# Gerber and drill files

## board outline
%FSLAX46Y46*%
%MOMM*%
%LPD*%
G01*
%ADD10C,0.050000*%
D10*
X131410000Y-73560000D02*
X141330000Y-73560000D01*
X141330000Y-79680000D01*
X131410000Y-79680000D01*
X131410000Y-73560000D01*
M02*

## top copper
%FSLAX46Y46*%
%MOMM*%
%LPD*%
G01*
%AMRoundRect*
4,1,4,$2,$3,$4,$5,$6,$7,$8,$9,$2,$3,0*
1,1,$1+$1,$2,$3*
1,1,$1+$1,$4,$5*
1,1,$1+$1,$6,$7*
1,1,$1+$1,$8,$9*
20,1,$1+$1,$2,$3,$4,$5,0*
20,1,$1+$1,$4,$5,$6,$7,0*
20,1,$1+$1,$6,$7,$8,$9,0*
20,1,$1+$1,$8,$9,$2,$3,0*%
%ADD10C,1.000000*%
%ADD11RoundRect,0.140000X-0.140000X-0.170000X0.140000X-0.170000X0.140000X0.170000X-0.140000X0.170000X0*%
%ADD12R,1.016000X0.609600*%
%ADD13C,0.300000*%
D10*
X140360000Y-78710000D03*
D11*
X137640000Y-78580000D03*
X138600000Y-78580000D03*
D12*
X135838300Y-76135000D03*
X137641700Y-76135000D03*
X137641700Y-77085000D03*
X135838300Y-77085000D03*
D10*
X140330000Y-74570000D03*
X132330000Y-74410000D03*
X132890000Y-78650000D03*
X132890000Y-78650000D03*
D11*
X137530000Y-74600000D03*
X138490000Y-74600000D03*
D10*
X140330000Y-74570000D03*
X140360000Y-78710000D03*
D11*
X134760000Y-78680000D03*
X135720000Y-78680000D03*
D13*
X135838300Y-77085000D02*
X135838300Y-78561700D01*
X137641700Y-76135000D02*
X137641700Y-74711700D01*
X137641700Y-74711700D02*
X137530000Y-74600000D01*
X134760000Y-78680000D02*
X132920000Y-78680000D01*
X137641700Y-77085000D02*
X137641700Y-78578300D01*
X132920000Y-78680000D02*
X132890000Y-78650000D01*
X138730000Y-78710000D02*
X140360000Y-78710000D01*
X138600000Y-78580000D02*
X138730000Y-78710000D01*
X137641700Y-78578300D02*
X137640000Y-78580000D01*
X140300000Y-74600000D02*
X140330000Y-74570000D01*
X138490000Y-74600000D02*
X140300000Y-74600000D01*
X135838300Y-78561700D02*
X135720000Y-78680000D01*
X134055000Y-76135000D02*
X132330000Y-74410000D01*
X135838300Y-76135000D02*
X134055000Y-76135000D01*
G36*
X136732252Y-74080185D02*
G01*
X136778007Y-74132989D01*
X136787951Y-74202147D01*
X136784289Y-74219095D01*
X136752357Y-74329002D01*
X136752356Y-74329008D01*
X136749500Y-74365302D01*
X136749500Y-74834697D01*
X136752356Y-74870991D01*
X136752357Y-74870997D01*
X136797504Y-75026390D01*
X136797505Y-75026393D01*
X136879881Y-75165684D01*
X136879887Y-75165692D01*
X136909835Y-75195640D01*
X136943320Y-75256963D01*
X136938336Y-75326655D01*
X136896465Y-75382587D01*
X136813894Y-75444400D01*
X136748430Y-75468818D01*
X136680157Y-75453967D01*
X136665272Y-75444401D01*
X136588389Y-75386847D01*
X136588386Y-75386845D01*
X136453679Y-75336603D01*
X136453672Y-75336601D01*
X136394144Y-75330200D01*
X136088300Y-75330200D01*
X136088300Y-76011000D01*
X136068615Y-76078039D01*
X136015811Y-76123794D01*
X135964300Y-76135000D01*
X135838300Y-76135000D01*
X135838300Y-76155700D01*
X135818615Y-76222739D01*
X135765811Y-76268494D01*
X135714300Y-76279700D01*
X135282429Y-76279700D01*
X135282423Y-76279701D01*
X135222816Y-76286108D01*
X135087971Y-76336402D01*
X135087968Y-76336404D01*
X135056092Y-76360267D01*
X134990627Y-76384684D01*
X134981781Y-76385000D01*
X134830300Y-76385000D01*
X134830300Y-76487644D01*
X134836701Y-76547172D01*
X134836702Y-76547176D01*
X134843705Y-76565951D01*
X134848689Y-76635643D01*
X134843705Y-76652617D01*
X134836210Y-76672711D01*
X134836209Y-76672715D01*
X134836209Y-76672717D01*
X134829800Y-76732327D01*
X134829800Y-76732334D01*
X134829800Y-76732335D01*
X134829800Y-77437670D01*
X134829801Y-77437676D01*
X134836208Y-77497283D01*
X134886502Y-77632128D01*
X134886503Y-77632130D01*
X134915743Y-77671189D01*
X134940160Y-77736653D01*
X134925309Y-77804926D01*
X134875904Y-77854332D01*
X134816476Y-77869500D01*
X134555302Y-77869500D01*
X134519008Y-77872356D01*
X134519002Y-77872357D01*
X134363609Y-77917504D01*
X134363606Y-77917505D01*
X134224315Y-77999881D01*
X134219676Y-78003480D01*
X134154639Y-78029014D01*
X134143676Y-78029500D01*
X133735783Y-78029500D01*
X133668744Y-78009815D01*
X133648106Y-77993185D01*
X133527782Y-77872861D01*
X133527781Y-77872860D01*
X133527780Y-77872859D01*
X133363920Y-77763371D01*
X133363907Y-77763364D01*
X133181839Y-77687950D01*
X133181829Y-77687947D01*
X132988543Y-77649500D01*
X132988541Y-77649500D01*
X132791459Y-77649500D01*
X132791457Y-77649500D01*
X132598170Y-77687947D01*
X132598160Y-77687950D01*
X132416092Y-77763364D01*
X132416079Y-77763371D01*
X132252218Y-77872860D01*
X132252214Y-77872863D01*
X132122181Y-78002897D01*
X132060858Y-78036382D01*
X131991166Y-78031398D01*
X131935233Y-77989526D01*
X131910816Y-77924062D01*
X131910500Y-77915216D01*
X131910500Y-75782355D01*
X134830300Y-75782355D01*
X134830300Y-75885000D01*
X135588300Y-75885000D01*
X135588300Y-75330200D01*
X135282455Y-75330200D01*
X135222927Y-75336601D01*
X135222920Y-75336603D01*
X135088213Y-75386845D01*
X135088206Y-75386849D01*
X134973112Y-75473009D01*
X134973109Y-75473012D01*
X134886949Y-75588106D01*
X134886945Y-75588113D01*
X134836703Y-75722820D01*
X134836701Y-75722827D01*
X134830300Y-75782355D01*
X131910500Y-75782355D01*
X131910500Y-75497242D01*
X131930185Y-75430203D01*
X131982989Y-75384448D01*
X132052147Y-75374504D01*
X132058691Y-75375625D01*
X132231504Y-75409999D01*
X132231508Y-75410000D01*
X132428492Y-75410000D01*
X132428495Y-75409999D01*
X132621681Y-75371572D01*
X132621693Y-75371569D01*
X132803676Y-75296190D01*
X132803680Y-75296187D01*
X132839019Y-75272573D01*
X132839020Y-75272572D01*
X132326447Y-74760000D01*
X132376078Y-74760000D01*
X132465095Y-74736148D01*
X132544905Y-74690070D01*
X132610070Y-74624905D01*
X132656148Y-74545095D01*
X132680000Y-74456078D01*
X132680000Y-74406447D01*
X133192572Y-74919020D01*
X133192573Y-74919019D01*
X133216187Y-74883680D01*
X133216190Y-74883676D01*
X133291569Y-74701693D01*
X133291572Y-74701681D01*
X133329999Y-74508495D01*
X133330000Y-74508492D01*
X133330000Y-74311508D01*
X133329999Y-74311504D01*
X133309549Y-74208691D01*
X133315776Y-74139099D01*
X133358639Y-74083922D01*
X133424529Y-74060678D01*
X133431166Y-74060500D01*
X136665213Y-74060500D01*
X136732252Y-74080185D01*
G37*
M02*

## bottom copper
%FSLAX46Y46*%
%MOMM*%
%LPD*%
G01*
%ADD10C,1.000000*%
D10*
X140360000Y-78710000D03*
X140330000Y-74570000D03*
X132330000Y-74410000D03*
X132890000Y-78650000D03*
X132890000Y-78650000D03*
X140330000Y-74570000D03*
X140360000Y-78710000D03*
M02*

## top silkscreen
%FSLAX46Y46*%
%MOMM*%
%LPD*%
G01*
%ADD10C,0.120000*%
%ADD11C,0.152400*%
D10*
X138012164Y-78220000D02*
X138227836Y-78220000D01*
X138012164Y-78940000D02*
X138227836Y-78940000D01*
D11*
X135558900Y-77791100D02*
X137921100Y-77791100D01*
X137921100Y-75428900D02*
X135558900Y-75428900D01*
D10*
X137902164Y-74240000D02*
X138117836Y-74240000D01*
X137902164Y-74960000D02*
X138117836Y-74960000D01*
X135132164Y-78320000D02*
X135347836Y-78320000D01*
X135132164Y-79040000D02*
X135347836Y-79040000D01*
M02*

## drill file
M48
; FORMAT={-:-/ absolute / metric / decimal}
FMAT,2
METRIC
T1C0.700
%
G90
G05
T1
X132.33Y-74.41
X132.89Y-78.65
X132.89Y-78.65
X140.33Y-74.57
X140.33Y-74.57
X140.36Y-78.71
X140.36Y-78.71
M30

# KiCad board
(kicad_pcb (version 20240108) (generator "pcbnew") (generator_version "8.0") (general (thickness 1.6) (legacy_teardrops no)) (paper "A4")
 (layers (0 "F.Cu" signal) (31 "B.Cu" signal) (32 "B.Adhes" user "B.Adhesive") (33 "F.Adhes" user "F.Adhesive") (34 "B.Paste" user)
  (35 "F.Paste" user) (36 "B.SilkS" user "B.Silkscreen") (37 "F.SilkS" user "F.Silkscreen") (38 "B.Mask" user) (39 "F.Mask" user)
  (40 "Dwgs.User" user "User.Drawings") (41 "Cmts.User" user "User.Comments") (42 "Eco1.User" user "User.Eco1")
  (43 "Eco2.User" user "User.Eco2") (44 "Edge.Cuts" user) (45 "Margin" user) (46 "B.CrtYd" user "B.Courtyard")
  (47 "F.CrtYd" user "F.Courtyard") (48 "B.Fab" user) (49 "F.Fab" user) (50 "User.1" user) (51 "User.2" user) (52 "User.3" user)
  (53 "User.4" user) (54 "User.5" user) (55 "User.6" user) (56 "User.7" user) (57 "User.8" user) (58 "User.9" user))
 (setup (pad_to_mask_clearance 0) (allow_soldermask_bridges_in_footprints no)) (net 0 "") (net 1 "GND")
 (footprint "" (layer "F.Cu") (at 140.36 78.71)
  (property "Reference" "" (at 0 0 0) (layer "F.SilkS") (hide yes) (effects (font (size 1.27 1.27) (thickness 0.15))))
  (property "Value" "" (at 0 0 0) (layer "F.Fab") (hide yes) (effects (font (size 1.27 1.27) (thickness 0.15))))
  (pad "1" thru_hole circle (at 0 0) (size 1 1) (drill 0.7) (layers "*.Cu" "*.Mask") (remove_unused_layers no)))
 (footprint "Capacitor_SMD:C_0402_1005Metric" (layer "F.Cu") (at 138.12 78.58)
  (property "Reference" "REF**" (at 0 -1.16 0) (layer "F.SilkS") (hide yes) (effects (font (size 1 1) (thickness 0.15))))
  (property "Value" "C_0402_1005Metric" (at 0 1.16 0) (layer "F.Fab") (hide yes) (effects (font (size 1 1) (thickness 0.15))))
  (fp_line (start -0.107836 -0.36) (end 0.107836 -0.36) (stroke (width 0.12) (type solid)) (layer "F.SilkS"))
  (fp_line (start -0.107836 0.36) (end 0.107836 0.36) (stroke (width 0.12) (type solid)) (layer "F.SilkS"))
  (pad "1" smd roundrect (at -0.48 0) (size 0.56 0.62) (layers "F.Cu" "F.Paste" "F.Mask") (roundrect_rratio 0.25))
  (pad "2" smd roundrect (at 0.48 0) (size 0.56 0.62) (layers "F.Cu" "F.Paste" "F.Mask") (roundrect_rratio 0.25)))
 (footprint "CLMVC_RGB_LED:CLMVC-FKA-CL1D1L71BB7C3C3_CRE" (layer "F.Cu") (at 136.74 76.61)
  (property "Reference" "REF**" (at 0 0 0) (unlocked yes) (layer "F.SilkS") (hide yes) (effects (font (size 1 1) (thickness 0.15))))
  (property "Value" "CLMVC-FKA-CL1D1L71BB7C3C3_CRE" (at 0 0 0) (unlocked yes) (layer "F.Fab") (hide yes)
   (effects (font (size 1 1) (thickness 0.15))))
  (fp_line (start -1.1811 1.1811) (end 1.1811 1.1811) (stroke (width 0.1524) (type solid)) (layer "F.SilkS"))
  (fp_line (start 1.1811 -1.1811) (end -1.1811 -1.1811) (stroke (width 0.1524) (type solid)) (layer "F.SilkS"))
  (pad "1" smd rect (at -0.9017 -0.475) (size 1.016 0.6096) (layers "F.Cu" "F.Paste" "F.Mask") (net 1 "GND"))
  (pad "2" smd rect (at 0.9017 -0.475) (size 1.016 0.6096) (layers "F.Cu" "F.Paste" "F.Mask"))
  (pad "3" smd rect (at 0.9017 0.475) (size 1.016 0.6096) (layers "F.Cu" "F.Paste" "F.Mask"))
  (pad "4" smd rect (at -0.9017 0.475) (size 1.016 0.6096) (layers "F.Cu" "F.Paste" "F.Mask")))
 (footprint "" (layer "F.Cu") (at 140.33 74.57)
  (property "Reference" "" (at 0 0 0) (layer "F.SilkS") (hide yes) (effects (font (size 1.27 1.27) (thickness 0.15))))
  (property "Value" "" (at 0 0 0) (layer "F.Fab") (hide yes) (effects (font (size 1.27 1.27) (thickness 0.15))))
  (pad "1" thru_hole circle (at 0 0) (size 1 1) (drill 0.7) (layers "*.Cu" "*.Mask") (remove_unused_layers no)))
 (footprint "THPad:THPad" (layer "F.Cu") (at 132.33 73.91)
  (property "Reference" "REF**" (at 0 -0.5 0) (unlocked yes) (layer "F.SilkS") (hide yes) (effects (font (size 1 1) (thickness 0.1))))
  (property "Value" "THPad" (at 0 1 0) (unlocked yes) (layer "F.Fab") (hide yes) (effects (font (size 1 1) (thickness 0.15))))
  (pad "1" thru_hole circle (at 0 0.5) (size 1 1) (drill 0.7) (layers "*.Cu" "*.Mask") (remove_unused_layers no) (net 1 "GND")))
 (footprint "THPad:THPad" (layer "F.Cu") (at 132.89 78.15)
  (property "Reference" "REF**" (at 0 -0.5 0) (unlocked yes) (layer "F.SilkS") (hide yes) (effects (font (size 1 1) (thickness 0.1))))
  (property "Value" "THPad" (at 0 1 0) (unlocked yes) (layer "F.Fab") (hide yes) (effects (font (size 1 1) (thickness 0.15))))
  (pad "1" thru_hole circle (at 0 0.5) (size 1 1) (drill 0.7) (layers "*.Cu" "*.Mask") (remove_unused_layers no)))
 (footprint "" (layer "F.Cu") (at 132.89 78.65)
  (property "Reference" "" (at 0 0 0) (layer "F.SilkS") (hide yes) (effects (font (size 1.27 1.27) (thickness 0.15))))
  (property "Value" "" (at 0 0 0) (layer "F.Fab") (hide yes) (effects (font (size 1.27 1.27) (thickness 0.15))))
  (pad "1" thru_hole circle (at 0 0) (size 1 1) (drill 0.7) (layers "*.Cu" "*.Mask") (remove_unused_layers no)))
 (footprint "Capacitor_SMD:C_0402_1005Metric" (layer "F.Cu") (at 138.01 74.6)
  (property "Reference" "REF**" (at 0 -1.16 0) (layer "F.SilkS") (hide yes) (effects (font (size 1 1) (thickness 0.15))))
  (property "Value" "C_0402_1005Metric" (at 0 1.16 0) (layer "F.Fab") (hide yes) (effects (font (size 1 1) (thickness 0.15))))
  (fp_line (start -0.107836 -0.36) (end 0.107836 -0.36) (stroke (width 0.12) (type solid)) (layer "F.SilkS"))
  (fp_line (start -0.107836 0.36) (end 0.107836 0.36) (stroke (width 0.12) (type solid)) (layer "F.SilkS"))
  (pad "1" smd roundrect (at -0.48 0) (size 0.56 0.62) (layers "F.Cu" "F.Paste" "F.Mask") (roundrect_rratio 0.25))
  (pad "2" smd roundrect (at 0.48 0) (size 0.56 0.62) (layers "F.Cu" "F.Paste" "F.Mask") (roundrect_rratio 0.25)))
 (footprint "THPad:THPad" (layer "F.Cu") (at 140.33 74.07)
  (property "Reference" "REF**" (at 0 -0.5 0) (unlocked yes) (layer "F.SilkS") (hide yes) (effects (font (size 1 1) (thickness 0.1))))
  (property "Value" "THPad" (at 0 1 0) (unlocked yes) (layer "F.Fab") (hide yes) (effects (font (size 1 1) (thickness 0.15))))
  (pad "1" thru_hole circle (at 0 0.5) (size 1 1) (drill 0.7) (layers "*.Cu" "*.Mask") (remove_unused_layers no)))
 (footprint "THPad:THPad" (layer "F.Cu") (at 140.36 78.21)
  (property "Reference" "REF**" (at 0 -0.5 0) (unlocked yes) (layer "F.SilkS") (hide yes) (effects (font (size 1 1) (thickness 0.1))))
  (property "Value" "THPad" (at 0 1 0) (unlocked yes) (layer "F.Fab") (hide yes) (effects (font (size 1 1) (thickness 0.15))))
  (pad "1" thru_hole circle (at 0 0.5) (size 1 1) (drill 0.7) (layers "*.Cu" "*.Mask") (remove_unused_layers no)))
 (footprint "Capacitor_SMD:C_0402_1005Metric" (layer "F.Cu") (at 135.24 78.68)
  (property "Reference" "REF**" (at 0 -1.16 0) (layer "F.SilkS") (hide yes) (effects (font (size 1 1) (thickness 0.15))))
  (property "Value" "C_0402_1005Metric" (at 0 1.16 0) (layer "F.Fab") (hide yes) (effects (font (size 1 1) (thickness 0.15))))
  (fp_line (start -0.107836 -0.36) (end 0.107836 -0.36) (stroke (width 0.12) (type solid)) (layer "F.SilkS"))
  (fp_line (start -0.107836 0.36) (end 0.107836 0.36) (stroke (width 0.12) (type solid)) (layer "F.SilkS"))
  (pad "1" smd roundrect (at -0.48 0) (size 0.56 0.62) (layers "F.Cu" "F.Paste" "F.Mask") (roundrect_rratio 0.25))
  (pad "2" smd roundrect (at 0.48 0) (size 0.56 0.62) (layers "F.Cu" "F.Paste" "F.Mask") (roundrect_rratio 0.25)))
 (gr_rect (start 131.41 73.56) (end 141.33 79.68) (stroke (width 0.05) (type default)) (fill none) (layer "Edge.Cuts"))
 (segment (start 135.8383 77.085) (end 135.8383 78.5617) (width 0.3) (layer "F.Cu") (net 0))
 (segment (start 137.6417 76.135) (end 137.6417 74.7117) (width 0.3) (layer "F.Cu") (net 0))
 (segment (start 137.6417 74.7117) (end 137.53 74.6) (width 0.3) (layer "F.Cu") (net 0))
 (segment (start 134.76 78.68) (end 132.92 78.68) (width 0.3) (layer "F.Cu") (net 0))
 (segment (start 137.6417 77.085) (end 137.6417 78.5783) (width 0.3) (layer "F.Cu") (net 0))
 (segment (start 132.92 78.68) (end 132.89 78.65) (width 0.3) (layer "F.Cu") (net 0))
 (segment (start 138.73 78.71) (end 140.36 78.71) (width 0.3) (layer "F.Cu") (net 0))
 (segment (start 138.6 78.58) (end 138.73 78.71) (width 0.3) (layer "F.Cu") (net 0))
 (segment (start 137.6417 78.5783) (end 137.64 78.58) (width 0.3) (layer "F.Cu") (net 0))
 (segment (start 140.3 74.6) (end 140.33 74.57) (width 0.3) (layer "F.Cu") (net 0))
 (segment (start 138.49 74.6) (end 140.3 74.6) (width 0.3) (layer "F.Cu") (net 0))
 (segment (start 135.8383 78.5617) (end 135.72 78.68) (width 0.3) (layer "F.Cu") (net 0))
 (segment (start 134.055 76.135) (end 132.33 74.41) (width 0.3) (layer "F.Cu") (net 1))
 (segment (start 135.8383 76.135) (end 134.055 76.135) (width 0.3) (layer "F.Cu") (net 1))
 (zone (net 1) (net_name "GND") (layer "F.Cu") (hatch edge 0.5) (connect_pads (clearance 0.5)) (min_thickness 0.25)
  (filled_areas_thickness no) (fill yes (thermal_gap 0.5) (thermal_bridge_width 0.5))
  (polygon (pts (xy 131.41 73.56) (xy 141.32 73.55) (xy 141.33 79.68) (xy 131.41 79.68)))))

